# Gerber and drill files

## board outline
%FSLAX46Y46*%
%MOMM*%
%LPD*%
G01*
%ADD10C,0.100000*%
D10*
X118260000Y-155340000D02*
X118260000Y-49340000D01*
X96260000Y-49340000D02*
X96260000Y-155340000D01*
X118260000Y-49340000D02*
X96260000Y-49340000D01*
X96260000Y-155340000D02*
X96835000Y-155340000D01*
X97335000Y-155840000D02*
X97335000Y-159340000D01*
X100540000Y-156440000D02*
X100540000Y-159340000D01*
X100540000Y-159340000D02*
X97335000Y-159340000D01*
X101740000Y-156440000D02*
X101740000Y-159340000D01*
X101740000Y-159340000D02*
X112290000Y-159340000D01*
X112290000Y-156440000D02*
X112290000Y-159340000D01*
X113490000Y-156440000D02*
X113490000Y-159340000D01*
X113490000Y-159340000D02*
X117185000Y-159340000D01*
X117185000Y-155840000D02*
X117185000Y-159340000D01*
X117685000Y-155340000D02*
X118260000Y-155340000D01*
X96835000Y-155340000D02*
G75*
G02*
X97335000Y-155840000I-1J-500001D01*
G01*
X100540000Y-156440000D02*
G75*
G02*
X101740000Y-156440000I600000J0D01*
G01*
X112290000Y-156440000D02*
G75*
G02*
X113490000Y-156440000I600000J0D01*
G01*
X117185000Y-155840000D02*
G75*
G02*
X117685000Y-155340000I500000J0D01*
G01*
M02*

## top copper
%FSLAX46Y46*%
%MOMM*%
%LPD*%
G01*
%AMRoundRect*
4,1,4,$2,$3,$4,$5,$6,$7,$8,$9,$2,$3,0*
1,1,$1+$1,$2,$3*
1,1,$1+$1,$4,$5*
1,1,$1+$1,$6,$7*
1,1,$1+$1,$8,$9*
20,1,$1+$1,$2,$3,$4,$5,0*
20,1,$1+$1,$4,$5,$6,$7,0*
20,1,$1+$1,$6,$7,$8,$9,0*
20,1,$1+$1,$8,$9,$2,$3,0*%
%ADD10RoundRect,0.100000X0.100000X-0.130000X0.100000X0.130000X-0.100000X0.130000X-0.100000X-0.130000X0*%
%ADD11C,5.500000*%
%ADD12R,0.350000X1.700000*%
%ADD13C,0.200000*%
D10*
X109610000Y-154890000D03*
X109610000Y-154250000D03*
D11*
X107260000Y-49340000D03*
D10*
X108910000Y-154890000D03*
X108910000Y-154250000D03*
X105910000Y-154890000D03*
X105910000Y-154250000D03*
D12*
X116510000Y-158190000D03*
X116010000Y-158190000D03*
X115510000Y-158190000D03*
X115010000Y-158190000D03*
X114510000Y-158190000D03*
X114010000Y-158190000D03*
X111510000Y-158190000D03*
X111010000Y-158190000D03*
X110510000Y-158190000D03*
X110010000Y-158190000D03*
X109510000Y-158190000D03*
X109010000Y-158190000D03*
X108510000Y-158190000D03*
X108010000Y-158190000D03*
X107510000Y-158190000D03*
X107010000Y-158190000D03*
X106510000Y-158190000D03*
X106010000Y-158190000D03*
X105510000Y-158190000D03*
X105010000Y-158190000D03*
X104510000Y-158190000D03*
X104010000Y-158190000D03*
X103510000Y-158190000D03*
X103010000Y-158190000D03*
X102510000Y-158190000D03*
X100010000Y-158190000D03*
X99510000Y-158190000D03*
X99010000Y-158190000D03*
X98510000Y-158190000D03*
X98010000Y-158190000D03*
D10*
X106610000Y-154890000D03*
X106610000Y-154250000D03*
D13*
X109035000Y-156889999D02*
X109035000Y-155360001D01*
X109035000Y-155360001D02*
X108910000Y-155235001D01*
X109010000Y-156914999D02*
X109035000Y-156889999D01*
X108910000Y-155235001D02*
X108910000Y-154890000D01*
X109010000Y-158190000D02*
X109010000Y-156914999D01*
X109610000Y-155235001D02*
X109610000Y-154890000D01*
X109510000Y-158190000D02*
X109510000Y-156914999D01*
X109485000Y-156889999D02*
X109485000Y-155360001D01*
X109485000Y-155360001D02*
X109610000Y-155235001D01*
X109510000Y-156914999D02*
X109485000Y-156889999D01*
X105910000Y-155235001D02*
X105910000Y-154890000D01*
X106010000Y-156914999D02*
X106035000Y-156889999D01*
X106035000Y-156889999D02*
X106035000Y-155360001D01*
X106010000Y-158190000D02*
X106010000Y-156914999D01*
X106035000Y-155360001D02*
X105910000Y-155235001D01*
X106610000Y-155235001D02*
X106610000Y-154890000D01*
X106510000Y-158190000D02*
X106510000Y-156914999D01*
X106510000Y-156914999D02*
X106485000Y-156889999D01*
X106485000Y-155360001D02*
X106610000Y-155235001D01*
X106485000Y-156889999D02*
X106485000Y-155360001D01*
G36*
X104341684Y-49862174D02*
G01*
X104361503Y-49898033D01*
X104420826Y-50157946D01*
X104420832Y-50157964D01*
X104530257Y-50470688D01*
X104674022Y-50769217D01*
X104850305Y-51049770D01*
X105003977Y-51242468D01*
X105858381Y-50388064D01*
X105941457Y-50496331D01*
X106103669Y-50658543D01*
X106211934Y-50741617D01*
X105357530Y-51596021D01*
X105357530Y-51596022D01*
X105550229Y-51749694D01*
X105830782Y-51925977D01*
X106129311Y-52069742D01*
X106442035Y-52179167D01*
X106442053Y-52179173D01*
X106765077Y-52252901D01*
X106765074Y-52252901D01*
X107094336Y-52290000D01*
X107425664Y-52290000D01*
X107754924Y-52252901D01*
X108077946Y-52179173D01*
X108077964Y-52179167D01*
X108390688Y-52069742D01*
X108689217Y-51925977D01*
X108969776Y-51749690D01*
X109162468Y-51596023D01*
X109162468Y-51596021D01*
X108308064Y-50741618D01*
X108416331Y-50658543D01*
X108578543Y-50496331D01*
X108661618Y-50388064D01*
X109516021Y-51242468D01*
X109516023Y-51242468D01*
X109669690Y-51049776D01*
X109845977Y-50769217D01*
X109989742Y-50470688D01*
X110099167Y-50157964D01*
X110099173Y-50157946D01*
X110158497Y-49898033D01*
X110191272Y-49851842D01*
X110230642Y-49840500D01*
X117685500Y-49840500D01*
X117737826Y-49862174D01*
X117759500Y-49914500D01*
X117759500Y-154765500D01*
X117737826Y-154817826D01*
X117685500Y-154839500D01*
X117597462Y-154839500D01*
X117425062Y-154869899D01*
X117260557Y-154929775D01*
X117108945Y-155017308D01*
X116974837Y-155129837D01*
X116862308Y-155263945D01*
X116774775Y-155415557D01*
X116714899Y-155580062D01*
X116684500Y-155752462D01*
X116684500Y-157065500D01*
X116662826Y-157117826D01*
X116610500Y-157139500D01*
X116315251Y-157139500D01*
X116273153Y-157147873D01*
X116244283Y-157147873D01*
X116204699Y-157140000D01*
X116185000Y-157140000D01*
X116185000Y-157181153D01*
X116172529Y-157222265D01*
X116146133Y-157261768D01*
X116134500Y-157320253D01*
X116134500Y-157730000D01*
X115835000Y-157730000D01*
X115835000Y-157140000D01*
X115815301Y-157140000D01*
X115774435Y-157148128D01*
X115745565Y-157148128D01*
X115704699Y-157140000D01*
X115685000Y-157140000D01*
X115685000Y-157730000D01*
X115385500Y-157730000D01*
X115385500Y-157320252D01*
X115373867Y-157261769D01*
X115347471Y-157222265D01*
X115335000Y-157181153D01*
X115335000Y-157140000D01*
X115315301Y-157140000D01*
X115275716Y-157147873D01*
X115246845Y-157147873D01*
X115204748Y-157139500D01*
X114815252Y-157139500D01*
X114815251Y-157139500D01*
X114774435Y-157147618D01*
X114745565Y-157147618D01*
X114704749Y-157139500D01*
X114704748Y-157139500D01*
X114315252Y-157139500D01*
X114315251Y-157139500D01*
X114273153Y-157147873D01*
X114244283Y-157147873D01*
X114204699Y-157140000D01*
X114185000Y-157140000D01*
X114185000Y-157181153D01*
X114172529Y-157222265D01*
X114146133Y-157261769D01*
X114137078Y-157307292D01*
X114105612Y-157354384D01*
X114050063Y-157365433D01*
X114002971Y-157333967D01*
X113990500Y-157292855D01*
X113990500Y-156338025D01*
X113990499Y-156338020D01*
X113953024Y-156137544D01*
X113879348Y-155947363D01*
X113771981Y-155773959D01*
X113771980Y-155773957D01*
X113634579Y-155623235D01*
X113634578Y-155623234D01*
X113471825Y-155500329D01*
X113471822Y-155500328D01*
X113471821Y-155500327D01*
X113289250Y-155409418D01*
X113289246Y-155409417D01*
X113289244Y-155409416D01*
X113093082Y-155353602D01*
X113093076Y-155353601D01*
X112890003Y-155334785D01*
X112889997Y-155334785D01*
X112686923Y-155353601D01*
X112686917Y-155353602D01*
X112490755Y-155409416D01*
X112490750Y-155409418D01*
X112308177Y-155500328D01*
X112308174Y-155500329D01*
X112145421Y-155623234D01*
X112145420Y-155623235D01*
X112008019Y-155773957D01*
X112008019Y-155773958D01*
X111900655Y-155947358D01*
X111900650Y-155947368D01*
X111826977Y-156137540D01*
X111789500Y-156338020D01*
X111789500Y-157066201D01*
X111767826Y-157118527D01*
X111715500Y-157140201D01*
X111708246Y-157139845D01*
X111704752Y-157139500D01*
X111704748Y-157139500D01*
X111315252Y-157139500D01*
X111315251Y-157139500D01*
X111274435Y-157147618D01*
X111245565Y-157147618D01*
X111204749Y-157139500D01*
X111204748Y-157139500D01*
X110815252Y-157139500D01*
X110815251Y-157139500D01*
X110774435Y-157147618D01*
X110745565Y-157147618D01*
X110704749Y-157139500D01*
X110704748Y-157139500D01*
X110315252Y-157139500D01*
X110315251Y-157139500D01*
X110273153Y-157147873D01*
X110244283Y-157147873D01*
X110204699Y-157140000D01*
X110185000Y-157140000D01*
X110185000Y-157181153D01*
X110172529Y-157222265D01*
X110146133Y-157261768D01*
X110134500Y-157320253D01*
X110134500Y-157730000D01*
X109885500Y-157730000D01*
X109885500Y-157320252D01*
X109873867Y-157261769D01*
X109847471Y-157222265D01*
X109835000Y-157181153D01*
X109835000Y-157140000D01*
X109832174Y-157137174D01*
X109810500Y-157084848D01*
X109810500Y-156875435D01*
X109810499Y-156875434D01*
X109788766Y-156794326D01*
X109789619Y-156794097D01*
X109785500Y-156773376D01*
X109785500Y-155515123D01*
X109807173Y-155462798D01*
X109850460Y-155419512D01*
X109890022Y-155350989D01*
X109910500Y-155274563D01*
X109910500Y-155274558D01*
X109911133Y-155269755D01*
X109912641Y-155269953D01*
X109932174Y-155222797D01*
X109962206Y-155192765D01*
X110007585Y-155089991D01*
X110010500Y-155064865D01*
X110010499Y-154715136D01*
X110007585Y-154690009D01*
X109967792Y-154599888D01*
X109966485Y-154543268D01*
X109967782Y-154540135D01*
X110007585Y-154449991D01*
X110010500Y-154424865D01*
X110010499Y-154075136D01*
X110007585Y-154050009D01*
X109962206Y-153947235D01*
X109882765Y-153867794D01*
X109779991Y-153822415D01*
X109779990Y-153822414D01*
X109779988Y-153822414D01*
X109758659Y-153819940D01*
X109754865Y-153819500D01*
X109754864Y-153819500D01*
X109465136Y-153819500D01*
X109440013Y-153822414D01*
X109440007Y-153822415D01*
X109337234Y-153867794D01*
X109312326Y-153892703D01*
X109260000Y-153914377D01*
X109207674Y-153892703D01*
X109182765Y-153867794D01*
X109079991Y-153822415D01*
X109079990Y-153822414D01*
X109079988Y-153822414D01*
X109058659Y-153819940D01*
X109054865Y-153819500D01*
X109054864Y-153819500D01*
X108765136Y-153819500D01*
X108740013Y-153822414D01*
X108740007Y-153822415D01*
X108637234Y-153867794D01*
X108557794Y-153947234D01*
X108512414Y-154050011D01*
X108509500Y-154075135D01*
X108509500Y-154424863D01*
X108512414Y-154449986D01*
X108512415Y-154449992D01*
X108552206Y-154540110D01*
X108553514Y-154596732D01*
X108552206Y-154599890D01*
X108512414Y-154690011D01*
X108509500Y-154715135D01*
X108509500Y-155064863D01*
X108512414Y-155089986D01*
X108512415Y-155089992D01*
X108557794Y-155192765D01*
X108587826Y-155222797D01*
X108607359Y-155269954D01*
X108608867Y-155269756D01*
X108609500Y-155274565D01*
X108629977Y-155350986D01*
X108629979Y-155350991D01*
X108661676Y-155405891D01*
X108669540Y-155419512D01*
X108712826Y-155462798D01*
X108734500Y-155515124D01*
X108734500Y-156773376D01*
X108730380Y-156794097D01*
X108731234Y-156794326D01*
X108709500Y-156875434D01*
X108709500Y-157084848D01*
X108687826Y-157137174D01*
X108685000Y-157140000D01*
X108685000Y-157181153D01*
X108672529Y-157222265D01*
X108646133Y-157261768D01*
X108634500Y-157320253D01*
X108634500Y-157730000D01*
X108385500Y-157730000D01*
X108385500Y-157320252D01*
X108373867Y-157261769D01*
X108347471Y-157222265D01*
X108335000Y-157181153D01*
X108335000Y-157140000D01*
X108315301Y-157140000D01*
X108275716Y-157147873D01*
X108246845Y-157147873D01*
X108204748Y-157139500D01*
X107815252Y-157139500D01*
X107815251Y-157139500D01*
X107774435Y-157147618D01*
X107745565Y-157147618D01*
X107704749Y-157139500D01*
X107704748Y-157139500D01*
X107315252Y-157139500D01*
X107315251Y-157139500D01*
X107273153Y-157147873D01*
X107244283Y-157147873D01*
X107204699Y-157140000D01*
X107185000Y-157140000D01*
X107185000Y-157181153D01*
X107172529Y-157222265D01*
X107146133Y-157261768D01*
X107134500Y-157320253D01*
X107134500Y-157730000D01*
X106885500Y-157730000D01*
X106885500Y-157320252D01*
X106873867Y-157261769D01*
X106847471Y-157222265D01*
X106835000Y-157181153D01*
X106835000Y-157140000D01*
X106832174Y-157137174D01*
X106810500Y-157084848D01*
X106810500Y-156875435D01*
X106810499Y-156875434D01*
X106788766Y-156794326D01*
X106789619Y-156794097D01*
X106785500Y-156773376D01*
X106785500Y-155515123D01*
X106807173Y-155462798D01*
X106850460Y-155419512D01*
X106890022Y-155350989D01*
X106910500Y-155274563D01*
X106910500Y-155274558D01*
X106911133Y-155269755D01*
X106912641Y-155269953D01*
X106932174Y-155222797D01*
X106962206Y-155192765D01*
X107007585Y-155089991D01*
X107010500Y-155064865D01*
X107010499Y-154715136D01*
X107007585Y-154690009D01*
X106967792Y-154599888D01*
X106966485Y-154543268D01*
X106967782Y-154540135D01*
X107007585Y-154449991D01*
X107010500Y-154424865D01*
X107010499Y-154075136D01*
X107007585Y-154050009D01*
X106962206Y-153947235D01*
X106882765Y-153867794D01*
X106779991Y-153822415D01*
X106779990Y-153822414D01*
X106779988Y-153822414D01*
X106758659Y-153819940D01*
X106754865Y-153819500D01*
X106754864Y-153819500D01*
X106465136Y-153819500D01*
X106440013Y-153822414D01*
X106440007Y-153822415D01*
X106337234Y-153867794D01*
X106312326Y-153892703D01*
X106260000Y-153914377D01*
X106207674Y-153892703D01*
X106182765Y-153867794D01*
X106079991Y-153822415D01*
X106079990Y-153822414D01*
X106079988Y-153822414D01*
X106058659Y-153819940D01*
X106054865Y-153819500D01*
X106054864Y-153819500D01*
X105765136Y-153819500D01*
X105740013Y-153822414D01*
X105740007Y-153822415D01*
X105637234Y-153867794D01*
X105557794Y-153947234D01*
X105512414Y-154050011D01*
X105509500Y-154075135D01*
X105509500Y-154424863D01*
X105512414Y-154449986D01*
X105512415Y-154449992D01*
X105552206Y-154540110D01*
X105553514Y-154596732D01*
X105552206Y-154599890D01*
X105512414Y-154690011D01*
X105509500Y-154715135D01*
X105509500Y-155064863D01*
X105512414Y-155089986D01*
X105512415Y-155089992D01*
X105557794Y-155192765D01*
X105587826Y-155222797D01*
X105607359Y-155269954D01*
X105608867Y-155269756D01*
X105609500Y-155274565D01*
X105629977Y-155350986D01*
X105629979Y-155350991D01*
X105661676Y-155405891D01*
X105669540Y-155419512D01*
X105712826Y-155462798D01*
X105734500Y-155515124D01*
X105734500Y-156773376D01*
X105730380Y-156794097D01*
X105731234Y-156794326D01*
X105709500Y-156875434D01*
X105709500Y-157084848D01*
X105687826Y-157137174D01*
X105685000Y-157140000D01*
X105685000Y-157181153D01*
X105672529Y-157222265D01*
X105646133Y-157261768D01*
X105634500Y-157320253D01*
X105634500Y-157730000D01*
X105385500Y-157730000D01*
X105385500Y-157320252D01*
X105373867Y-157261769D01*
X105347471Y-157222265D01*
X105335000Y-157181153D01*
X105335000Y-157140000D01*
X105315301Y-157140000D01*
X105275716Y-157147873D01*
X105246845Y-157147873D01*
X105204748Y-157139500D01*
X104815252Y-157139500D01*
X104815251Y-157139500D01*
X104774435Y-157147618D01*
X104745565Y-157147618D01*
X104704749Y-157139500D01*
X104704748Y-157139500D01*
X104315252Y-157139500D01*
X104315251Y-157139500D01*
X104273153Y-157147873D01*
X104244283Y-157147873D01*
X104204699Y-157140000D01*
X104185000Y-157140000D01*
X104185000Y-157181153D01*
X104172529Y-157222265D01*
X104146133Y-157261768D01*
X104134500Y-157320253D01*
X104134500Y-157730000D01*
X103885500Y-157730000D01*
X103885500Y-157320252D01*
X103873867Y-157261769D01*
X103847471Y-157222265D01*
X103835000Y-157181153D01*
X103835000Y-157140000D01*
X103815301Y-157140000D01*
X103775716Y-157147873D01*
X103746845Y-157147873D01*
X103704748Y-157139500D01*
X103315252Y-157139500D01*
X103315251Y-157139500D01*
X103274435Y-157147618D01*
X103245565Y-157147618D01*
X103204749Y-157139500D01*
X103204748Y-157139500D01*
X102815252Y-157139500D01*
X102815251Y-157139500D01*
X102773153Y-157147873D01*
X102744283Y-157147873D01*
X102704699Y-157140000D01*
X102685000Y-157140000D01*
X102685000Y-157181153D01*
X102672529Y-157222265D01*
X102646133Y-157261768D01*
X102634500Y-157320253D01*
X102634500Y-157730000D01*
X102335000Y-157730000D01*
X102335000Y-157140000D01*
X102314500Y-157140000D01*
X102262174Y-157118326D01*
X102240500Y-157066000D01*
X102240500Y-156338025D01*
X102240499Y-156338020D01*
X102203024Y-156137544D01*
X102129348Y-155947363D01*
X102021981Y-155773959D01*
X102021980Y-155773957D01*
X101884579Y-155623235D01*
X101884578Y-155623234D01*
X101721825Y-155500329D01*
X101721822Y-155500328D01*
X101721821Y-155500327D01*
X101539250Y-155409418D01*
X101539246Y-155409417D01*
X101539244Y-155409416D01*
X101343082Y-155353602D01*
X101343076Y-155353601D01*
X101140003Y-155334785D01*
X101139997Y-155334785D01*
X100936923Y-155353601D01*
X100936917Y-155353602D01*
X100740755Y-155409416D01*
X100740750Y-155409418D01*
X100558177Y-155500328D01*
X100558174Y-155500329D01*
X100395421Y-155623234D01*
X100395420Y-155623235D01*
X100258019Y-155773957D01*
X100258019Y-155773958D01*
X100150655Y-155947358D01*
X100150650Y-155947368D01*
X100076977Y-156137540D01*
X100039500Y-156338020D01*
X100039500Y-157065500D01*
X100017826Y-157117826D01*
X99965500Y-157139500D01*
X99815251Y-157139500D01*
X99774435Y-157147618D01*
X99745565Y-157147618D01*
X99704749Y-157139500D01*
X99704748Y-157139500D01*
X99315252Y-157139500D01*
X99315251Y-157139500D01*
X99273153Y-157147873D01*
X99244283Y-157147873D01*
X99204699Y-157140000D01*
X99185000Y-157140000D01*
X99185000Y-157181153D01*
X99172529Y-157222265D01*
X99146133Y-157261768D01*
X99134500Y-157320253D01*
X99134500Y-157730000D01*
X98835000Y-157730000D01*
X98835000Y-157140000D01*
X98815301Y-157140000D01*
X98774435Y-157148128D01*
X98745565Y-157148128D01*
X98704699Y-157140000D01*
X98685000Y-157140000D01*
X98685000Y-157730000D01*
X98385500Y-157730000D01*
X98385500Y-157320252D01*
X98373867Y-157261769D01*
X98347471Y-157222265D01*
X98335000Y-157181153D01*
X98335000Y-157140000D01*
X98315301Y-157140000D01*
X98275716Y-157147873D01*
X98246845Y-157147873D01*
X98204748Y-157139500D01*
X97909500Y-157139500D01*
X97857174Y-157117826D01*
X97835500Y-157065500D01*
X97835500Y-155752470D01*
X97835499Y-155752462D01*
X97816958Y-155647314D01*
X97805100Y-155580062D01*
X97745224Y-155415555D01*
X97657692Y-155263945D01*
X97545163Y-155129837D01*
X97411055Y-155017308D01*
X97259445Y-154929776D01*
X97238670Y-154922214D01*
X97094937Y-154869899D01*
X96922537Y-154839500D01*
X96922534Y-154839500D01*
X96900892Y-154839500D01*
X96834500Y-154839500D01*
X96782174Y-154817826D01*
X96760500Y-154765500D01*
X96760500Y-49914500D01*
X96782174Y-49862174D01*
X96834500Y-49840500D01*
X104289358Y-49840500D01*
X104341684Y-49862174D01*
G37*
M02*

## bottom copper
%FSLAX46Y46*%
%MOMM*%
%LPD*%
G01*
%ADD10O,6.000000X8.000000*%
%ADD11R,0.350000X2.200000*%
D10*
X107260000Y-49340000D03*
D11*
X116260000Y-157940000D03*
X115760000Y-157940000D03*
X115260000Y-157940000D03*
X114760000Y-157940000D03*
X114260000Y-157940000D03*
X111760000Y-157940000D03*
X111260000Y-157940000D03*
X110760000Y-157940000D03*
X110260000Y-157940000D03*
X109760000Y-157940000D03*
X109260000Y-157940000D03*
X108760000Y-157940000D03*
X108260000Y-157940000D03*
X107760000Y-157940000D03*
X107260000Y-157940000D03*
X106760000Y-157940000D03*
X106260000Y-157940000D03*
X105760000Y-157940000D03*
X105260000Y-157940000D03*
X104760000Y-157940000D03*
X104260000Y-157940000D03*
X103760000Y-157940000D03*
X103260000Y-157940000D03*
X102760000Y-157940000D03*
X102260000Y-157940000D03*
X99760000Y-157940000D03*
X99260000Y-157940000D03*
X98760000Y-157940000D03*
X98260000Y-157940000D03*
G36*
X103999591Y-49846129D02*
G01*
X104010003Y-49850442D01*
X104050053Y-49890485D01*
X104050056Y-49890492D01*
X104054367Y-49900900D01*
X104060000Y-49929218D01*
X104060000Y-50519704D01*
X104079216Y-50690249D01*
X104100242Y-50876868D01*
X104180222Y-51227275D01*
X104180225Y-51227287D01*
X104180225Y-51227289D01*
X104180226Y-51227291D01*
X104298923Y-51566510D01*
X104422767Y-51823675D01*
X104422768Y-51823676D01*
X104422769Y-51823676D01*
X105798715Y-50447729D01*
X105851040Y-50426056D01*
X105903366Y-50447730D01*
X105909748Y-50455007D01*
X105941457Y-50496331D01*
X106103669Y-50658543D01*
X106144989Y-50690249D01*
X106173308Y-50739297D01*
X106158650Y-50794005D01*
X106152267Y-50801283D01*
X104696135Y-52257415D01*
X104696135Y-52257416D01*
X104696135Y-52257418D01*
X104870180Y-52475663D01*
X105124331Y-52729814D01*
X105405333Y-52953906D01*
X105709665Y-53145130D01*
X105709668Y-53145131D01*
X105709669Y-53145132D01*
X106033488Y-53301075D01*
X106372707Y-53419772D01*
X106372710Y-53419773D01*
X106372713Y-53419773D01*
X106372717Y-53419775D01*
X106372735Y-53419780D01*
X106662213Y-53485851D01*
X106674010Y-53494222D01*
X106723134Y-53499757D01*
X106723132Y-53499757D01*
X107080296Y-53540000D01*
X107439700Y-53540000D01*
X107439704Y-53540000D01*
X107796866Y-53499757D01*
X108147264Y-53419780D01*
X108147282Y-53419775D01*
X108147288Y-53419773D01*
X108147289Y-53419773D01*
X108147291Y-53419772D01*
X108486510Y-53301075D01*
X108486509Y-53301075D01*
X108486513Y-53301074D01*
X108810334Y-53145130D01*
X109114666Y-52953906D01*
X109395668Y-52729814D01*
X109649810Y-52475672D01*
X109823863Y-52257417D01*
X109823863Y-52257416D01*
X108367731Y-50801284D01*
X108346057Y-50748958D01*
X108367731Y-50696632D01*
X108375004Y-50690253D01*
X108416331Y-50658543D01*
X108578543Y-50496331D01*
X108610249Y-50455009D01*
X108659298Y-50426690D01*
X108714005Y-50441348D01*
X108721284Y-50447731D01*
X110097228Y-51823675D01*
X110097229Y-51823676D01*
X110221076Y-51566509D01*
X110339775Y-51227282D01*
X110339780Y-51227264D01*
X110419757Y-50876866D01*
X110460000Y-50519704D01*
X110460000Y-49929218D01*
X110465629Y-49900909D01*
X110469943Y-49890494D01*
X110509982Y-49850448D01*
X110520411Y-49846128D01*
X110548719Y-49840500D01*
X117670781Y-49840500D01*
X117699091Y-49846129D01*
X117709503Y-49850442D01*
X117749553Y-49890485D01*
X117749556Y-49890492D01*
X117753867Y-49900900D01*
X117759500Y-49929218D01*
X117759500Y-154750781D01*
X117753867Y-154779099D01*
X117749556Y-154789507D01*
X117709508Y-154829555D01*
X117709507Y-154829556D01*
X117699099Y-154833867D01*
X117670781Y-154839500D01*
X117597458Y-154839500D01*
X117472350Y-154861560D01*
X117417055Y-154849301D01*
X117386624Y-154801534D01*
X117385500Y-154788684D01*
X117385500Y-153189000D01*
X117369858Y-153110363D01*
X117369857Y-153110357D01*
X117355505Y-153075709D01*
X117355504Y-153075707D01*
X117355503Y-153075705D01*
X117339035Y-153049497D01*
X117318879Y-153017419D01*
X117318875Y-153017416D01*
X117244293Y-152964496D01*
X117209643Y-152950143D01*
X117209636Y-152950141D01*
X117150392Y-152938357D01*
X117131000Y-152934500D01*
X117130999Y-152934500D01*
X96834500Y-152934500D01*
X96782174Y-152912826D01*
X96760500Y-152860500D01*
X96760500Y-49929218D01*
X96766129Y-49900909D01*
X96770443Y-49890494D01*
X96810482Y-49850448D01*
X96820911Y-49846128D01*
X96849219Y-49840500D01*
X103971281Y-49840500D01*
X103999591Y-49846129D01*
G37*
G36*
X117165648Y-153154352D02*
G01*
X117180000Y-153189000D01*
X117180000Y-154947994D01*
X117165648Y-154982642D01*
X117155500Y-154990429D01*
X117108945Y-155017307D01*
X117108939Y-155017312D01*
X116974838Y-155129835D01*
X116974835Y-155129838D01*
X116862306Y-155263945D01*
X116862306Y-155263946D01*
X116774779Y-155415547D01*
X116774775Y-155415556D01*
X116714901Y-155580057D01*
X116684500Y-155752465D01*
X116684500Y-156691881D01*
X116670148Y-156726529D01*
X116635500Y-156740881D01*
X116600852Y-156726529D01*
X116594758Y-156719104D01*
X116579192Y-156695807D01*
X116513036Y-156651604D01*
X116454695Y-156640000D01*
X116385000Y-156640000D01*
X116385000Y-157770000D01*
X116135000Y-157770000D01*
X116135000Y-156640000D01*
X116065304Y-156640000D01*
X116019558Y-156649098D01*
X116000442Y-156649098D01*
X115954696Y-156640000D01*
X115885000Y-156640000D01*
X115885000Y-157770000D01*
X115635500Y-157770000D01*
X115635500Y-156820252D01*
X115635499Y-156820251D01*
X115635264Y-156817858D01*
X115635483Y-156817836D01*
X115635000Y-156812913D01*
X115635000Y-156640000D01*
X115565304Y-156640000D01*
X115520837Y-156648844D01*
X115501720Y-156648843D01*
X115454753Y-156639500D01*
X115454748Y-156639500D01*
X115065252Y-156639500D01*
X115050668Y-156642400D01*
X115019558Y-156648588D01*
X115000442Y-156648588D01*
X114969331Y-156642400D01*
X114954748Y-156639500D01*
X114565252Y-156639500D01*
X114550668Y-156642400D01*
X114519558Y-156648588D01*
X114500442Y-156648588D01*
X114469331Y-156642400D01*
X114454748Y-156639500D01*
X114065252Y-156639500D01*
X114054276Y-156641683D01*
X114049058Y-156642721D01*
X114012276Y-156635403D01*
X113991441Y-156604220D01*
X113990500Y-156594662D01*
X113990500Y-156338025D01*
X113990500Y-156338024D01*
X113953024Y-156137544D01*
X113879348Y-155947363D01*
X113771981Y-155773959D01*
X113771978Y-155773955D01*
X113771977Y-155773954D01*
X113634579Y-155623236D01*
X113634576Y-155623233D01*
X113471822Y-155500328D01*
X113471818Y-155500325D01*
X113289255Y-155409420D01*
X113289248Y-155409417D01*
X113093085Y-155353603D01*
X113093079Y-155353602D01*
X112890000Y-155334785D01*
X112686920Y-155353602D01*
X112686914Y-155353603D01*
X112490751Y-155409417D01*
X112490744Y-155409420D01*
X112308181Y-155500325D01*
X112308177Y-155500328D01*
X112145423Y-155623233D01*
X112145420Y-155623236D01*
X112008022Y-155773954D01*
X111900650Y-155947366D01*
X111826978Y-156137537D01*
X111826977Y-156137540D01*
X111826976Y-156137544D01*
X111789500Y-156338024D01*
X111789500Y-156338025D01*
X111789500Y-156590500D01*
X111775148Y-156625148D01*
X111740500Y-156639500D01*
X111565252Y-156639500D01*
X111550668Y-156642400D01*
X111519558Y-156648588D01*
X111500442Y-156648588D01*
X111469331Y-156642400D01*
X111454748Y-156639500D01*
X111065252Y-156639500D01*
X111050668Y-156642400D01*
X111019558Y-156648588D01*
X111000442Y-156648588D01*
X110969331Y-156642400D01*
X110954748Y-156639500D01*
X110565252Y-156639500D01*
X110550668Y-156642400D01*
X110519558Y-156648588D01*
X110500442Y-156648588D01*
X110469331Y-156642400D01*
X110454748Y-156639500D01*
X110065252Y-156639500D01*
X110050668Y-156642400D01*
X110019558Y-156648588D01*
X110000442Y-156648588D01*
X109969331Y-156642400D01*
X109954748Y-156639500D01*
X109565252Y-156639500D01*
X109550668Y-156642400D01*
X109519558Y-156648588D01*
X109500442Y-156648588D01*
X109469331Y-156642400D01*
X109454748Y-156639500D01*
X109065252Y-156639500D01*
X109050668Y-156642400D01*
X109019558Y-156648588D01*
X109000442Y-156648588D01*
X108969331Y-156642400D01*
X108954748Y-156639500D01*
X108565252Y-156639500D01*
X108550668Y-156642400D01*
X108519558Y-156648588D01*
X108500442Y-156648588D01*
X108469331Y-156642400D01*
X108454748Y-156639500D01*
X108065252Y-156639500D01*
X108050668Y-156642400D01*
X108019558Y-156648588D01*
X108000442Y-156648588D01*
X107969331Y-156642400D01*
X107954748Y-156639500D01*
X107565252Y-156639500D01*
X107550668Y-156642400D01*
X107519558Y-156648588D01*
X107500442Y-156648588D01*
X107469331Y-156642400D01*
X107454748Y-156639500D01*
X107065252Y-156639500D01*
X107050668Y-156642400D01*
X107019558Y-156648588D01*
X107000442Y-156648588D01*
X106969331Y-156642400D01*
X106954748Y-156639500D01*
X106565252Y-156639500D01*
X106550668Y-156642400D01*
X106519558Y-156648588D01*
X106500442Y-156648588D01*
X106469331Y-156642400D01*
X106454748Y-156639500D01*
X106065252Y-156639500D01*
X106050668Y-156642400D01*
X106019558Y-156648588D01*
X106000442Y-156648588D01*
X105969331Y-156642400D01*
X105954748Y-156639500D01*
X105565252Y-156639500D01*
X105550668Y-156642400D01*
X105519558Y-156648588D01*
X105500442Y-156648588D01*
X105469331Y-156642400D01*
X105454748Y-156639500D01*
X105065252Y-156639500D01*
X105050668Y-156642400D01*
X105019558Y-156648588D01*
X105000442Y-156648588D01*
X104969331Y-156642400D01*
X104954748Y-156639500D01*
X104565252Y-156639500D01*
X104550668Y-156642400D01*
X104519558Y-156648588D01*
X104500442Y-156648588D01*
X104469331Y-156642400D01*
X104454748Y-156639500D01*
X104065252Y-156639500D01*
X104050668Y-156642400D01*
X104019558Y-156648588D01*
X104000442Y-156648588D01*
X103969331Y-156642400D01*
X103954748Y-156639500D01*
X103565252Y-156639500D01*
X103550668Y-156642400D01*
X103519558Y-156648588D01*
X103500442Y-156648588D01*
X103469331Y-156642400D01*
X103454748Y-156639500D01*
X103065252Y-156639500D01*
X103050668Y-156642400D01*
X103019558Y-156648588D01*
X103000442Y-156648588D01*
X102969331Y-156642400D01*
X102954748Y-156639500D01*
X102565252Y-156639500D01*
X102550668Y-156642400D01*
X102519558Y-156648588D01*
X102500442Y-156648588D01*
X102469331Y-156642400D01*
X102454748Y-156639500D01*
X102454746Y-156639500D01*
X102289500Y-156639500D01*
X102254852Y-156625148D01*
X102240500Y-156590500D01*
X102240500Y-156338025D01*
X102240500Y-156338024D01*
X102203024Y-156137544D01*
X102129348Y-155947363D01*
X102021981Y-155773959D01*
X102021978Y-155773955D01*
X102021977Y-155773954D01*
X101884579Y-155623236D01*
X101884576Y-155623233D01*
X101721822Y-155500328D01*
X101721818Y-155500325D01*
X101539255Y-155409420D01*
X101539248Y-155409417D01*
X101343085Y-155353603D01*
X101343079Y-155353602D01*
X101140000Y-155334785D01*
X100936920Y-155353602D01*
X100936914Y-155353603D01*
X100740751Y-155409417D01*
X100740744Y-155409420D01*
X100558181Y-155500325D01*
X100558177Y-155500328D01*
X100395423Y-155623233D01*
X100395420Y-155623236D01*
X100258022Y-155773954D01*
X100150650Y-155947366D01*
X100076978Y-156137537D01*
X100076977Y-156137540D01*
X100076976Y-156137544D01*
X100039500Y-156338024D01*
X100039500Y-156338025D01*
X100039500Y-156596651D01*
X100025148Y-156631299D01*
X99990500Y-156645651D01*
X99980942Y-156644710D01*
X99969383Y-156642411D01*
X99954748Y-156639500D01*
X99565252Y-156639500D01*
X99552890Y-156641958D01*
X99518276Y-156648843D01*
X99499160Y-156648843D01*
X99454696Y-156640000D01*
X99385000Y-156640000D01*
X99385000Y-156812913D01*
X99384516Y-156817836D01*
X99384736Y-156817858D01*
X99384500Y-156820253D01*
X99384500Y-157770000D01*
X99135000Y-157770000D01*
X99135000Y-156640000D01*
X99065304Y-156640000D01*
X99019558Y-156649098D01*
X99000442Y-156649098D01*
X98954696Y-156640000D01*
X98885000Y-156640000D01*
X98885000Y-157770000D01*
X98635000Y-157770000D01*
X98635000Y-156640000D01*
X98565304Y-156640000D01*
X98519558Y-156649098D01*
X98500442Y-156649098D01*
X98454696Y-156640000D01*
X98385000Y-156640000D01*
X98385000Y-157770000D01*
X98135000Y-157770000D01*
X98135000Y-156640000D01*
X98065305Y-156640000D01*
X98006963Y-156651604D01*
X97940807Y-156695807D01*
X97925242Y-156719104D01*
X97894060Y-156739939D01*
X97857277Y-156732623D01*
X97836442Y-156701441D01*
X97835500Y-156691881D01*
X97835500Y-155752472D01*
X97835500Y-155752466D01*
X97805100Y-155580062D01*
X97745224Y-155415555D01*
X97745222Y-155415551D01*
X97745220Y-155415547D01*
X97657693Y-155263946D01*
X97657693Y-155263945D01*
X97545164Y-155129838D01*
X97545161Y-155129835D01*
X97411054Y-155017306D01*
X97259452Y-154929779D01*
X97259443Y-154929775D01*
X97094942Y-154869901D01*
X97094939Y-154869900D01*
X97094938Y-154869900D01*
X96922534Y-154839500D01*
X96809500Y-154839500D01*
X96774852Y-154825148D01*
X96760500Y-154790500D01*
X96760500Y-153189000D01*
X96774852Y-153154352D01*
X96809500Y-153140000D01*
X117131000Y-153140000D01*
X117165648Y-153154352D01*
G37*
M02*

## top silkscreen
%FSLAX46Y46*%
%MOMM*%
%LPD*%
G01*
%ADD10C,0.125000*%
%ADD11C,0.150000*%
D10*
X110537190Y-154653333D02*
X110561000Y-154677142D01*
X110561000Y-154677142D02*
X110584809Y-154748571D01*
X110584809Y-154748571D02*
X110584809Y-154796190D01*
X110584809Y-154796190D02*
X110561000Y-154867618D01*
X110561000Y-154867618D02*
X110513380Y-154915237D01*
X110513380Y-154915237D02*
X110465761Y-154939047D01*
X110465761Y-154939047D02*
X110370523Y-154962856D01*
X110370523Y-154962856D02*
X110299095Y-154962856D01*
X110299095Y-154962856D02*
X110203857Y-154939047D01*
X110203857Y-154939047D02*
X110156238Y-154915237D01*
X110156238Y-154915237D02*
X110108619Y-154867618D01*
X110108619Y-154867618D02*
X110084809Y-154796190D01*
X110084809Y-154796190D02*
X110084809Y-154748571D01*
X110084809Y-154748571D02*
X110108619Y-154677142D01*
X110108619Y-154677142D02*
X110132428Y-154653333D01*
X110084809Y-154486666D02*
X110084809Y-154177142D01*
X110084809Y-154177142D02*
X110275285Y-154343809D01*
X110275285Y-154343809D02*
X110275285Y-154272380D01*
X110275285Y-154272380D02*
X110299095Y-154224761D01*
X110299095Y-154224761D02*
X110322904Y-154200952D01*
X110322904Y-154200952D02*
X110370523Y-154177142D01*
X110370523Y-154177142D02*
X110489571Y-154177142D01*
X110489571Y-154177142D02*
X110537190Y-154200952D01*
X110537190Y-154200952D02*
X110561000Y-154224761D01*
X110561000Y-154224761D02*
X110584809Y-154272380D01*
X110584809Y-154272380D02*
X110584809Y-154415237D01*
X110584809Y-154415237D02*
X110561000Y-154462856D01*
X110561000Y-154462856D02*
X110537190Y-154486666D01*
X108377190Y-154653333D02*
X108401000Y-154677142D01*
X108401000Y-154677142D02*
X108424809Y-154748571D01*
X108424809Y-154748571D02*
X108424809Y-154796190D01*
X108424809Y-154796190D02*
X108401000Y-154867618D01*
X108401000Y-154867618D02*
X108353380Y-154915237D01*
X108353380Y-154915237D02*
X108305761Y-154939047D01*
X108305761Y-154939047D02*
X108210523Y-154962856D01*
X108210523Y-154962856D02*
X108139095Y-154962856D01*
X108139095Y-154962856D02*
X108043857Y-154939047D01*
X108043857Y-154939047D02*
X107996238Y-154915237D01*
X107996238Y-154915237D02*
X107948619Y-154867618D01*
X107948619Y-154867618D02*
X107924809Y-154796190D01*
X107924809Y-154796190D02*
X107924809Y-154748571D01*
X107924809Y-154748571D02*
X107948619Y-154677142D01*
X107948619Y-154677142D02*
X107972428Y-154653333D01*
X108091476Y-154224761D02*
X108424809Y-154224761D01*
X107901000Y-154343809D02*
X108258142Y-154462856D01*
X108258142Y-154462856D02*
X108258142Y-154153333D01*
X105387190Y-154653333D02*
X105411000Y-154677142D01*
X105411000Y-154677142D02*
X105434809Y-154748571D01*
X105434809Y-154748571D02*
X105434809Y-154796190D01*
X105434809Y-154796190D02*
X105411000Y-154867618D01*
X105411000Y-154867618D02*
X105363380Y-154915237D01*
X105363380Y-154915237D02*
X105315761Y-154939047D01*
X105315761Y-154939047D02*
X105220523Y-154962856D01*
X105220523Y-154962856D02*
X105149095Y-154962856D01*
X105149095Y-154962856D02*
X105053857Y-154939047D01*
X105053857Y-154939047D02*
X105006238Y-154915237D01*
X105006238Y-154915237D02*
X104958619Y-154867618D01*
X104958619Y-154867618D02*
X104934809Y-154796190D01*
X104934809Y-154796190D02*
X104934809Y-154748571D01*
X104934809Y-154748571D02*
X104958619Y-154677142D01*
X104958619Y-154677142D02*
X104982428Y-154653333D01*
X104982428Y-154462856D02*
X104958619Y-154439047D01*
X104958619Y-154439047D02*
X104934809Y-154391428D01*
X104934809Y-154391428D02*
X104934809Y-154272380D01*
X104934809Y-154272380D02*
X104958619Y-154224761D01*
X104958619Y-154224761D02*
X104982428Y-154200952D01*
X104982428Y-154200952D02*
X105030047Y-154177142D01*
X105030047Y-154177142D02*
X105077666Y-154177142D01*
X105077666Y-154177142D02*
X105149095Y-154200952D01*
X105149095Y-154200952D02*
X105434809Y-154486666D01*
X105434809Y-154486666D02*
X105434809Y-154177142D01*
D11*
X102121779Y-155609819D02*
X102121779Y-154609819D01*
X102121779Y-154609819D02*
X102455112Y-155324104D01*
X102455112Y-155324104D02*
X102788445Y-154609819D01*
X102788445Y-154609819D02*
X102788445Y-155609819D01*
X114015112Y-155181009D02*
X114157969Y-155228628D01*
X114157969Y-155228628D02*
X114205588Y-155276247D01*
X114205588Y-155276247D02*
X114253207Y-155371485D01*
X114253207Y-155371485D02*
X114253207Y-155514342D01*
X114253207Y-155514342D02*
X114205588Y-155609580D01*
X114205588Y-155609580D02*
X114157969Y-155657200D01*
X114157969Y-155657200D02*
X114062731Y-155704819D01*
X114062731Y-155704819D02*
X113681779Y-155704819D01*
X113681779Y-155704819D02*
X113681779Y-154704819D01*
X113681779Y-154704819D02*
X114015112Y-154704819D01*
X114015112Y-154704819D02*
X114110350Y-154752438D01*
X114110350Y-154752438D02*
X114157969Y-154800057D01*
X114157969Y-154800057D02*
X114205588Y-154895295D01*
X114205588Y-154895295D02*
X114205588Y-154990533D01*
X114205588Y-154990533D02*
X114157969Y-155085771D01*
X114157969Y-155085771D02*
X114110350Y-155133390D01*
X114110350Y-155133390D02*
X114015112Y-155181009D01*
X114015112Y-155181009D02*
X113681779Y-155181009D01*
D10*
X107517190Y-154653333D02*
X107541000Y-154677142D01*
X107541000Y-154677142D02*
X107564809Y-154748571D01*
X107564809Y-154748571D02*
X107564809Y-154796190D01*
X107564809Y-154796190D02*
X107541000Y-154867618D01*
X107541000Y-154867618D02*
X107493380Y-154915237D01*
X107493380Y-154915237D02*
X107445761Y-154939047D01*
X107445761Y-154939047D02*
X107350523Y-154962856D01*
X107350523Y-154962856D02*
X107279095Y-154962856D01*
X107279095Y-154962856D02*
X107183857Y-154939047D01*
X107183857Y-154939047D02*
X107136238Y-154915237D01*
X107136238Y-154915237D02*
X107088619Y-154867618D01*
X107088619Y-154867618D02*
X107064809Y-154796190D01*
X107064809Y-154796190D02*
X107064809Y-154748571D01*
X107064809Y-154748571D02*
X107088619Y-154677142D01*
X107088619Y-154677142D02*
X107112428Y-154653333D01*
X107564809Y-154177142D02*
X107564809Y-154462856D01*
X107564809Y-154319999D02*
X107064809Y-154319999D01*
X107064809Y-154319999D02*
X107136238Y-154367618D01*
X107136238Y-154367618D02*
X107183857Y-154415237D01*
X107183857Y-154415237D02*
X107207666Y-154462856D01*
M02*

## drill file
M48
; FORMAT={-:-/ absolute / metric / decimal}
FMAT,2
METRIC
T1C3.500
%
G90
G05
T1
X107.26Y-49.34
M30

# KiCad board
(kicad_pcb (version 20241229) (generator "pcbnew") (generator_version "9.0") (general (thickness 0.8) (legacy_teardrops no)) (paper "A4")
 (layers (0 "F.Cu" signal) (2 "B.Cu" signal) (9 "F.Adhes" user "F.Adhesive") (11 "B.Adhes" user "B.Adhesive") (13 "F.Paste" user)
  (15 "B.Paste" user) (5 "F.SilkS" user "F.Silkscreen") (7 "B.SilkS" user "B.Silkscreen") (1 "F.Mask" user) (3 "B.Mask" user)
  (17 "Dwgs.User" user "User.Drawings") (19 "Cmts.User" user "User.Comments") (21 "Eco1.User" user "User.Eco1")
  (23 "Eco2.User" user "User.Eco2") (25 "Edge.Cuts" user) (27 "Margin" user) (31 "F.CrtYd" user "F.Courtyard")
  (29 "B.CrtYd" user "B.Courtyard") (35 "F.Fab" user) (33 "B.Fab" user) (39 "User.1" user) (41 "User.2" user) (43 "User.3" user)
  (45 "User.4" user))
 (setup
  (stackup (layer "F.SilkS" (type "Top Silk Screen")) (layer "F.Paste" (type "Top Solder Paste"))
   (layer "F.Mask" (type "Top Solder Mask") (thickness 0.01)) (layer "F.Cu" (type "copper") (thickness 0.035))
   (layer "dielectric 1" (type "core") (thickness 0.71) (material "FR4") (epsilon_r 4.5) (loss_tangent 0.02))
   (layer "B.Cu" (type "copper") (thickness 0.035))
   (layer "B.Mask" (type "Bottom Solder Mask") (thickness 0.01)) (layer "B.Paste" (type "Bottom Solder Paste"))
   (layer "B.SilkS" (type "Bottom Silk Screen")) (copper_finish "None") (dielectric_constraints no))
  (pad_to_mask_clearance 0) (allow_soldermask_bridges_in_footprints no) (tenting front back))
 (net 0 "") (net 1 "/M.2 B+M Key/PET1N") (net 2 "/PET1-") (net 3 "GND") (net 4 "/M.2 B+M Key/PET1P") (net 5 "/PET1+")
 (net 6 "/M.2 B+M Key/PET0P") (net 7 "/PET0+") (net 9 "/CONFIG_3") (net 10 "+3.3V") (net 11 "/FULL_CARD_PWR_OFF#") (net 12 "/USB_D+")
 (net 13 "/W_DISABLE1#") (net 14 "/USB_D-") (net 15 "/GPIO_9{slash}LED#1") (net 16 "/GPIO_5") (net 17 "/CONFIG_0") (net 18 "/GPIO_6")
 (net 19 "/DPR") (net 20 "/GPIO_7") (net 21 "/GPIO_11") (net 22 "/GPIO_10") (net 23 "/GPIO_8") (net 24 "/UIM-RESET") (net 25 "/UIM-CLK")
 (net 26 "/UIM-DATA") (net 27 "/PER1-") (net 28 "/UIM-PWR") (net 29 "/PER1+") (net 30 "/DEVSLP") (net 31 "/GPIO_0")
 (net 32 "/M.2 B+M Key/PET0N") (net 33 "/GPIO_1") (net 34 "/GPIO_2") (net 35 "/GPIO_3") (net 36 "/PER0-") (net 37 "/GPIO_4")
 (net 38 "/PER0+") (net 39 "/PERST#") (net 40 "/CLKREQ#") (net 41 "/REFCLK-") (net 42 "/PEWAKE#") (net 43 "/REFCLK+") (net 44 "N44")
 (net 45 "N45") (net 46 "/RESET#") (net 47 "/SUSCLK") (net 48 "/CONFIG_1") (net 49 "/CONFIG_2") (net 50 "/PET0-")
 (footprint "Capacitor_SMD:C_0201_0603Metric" (layer "F.Cu") (at 109.61 154.57 90)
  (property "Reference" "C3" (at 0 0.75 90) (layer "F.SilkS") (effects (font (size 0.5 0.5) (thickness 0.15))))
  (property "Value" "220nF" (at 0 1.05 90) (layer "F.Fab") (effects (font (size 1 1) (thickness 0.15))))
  (pad "" smd roundrect (at -0.345 0 90) (size 0.318 0.36) (layers "F.Paste") (roundrect_rratio 0.25))
  (pad "" smd roundrect (at 0.345 0 90) (size 0.318 0.36) (layers "F.Paste") (roundrect_rratio 0.25))
  (pad "1" smd roundrect (at -0.32 0 90) (size 0.46 0.4) (layers "F.Cu" "F.Mask") (roundrect_rratio 0.25) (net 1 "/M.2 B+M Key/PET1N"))
  (pad "2" smd roundrect (at 0.32 0 90) (size 0.46 0.4) (layers "F.Cu" "F.Mask") (roundrect_rratio 0.25) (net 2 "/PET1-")))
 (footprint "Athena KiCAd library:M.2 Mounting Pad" (layer "F.Cu") (at 107.26 49.34)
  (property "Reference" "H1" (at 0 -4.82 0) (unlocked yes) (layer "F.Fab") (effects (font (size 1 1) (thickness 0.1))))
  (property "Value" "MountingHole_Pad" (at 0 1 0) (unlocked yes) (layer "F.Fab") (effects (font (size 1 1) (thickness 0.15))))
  (pad "1" thru_hole circle (at 0 0) (size 5.5 5.5) (drill 3.5) (layers "*.Cu" "*.Mask") (remove_unused_layers no) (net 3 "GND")
   (padstack (mode front_inner_back)
    (layer "Inner" (shape circle) (size 5.5 5.5) (zone_connect -1))
    (layer "B.Cu" (shape oval) (size 6 8) (thermal_bridge_angle 45) (zone_connect -1)))))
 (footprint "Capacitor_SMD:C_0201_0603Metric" (layer "F.Cu") (at 108.91 154.57 90)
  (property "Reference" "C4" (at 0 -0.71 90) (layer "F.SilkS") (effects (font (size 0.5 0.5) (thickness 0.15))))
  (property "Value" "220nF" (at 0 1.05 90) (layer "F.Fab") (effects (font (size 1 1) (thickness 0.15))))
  (pad "" smd roundrect (at -0.345 0 90) (size 0.318 0.36) (layers "F.Paste") (roundrect_rratio 0.25))
  (pad "" smd roundrect (at 0.345 0 90) (size 0.318 0.36) (layers "F.Paste") (roundrect_rratio 0.25))
  (pad "1" smd roundrect (at -0.32 0 90) (size 0.46 0.4) (layers "F.Cu" "F.Mask") (roundrect_rratio 0.25) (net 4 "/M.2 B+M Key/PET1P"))
  (pad "2" smd roundrect (at 0.32 0 90) (size 0.46 0.4) (layers "F.Cu" "F.Mask") (roundrect_rratio 0.25) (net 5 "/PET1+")))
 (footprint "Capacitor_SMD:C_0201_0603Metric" (layer "F.Cu") (at 105.91 154.57 90)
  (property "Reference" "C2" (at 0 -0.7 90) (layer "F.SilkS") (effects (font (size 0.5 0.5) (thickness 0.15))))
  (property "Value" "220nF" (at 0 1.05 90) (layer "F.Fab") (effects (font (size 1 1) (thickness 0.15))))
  (pad "" smd roundrect (at -0.345 0 90) (size 0.318 0.36) (layers "F.Paste") (roundrect_rratio 0.25))
  (pad "" smd roundrect (at 0.345 0 90) (size 0.318 0.36) (layers "F.Paste") (roundrect_rratio 0.25))
  (pad "1" smd roundrect (at -0.32 0 90) (size 0.46 0.4) (layers "F.Cu" "F.Mask") (roundrect_rratio 0.25) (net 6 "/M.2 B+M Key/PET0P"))
  (pad "2" smd roundrect (at 0.32 0 90) (size 0.46 0.4) (layers "F.Cu" "F.Mask") (roundrect_rratio 0.25) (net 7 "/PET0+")))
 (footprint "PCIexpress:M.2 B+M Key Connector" (layer "F.Cu") (at 107.26 158.23)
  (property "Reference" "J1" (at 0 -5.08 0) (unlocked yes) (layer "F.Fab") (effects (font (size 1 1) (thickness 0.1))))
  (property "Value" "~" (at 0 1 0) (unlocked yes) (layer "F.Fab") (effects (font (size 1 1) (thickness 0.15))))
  (fp_line (start -11 -2.89) (end -10.425 -2.89) (stroke (width 0.1) (type default)) (layer "Edge.Cuts") (net 8))
  (fp_line (start -9.925 -2.39) (end -9.925 1.11) (stroke (width 0.1) (type default)) (layer "Edge.Cuts") (net 8))
  (fp_line (start -6.72 -1.79) (end -6.72 1.11) (stroke (width 0.1) (type default)) (layer "Edge.Cuts") (net 8))
  (fp_line (start -6.72 1.11) (end -9.925 1.11) (stroke (width 0.1) (type default)) (layer "Edge.Cuts") (net 8))
  (fp_line (start -5.52 -1.79) (end -5.52 1.11) (stroke (width 0.1) (type default)) (layer "Edge.Cuts") (net 8))
  (fp_line (start -5.52 1.11) (end 5.03 1.11) (stroke (width 0.1) (type default)) (layer "Edge.Cuts") (net 8))
  (fp_line (start 5.03 -1.79) (end 5.03 1.11) (stroke (width 0.1) (type default)) (layer "Edge.Cuts") (net 8))
  (fp_line (start 6.23 -1.79) (end 6.23 1.11) (stroke (width 0.1) (type default)) (layer "Edge.Cuts") (net 8))
  (fp_line (start 6.23 1.11) (end 9.925 1.11) (stroke (width 0.1) (type default)) (layer "Edge.Cuts") (net 8))
  (fp_line (start 9.925 -2.39) (end 9.925 1.11) (stroke (width 0.1) (type default)) (layer "Edge.Cuts") (net 8))
  (fp_line (start 10.425 -2.89) (end 11 -2.89) (stroke (width 0.1) (type default)) (layer "Edge.Cuts") (net 8))
  (fp_arc (start -10.425 -2.89) (mid -10.071447 -2.743553) (end -9.925 -2.39) (stroke (width 0.1) (type default)) (layer "Edge.Cuts")
   (net 8))
  (fp_arc (start -6.72 -1.79) (mid -6.12 -2.39) (end -5.52 -1.79) (stroke (width 0.1) (type default)) (layer "Edge.Cuts") (net 8))
  (fp_arc (start 5.03 -1.79) (mid 5.63 -2.39) (end 6.23 -1.79) (stroke (width 0.1) (type default)) (layer "Edge.Cuts") (net 8))
  (fp_arc (start 9.925 -2.39) (mid 10.071447 -2.743553) (end 10.425 -2.89) (stroke (width 0.1) (type default)) (layer "Edge.Cuts") (net 8))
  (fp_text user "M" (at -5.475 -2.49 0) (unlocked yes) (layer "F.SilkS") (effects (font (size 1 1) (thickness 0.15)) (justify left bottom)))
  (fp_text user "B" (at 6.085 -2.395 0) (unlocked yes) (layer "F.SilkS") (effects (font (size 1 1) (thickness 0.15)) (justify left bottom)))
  (pad "1" smd rect (at 9.25 -0.04 180) (size 0.35 1.7) (layers "F.Cu") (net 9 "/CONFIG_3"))
  (pad "2" smd rect (at 9 -0.29 180) (size 0.35 2.2) (layers "B.Cu") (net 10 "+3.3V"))
  (pad "3" smd rect (at 8.75 -0.04 180) (size 0.35 1.7) (layers "F.Cu") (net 3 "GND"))
  (pad "4" smd rect (at 8.5 -0.29 180) (size 0.35 2.2) (layers "B.Cu") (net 10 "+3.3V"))
  (pad "5" smd rect (at 8.25 -0.04 180) (size 0.35 1.7) (layers "F.Cu") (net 3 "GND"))
  (pad "6" smd rect (at 8 -0.29 180) (size 0.35 2.2) (layers "B.Cu") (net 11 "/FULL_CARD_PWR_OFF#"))
  (pad "7" smd rect (at 7.75 -0.04 180) (size 0.35 1.7) (layers "F.Cu") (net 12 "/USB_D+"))
  (pad "8" smd rect (at 7.5 -0.29 180) (size 0.35 2.2) (layers "B.Cu") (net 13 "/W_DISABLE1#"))
  (pad "9" smd rect (at 7.25 -0.04 180) (size 0.35 1.7) (layers "F.Cu") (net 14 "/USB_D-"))
  (pad "10" smd rect (at 7 -0.29 180) (size 0.35 2.2) (layers "B.Cu") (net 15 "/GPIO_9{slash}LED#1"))
  (pad "11" smd rect (at 6.75 -0.04 180) (size 0.35 1.7) (layers "F.Cu") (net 3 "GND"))
  (pad "20" smd rect (at 4.5 -0.29 180) (size 0.35 2.2) (layers "B.Cu") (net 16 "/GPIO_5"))
  (pad "21" smd rect (at 4.25 -0.04 180) (size 0.35 1.7) (layers "F.Cu") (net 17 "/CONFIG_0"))
  (pad "22" smd rect (at 4 -0.29 180) (size 0.35 2.2) (layers "B.Cu") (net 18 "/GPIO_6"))
  (pad "23" smd rect (at 3.75 -0.04 180) (size 0.35 1.7) (layers "F.Cu") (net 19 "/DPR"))
  (pad "24" smd rect (at 3.5 -0.29 180) (size 0.35 2.2) (layers "B.Cu") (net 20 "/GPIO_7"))
  (pad "25" smd rect (at 3.25 -0.04 180) (size 0.35 1.7) (layers "F.Cu") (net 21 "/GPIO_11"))
  (pad "26" smd rect (at 3 -0.29 180) (size 0.35 2.2) (layers "B.Cu") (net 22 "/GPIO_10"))
  (pad "27" smd rect (at 2.75 -0.04 180) (size 0.35 1.7) (layers "F.Cu") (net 3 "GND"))
  (pad "28" smd rect (at 2.5 -0.29 180) (size 0.35 2.2) (layers "B.Cu") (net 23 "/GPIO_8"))
  (pad "29" smd rect (at 2.25 -0.04 180) (size 0.35 1.7) (layers "F.Cu") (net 1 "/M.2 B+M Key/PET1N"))
  (pad "30" smd rect (at 2 -0.29 180) (size 0.35 2.2) (layers "B.Cu") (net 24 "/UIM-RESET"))
  (pad "31" smd rect (at 1.75 -0.04 180) (size 0.35 1.7) (layers "F.Cu") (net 4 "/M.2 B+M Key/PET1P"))
  (pad "32" smd rect (at 1.5 -0.29 180) (size 0.35 2.2) (layers "B.Cu") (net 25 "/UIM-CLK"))
  (pad "33" smd rect (at 1.25 -0.04 180) (size 0.35 1.7) (layers "F.Cu") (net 3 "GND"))
  (pad "34" smd rect (at 1 -0.29 180) (size 0.35 2.2) (layers "B.Cu") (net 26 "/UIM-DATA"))
  (pad "35" smd rect (at 0.75 -0.04 180) (size 0.35 1.7) (layers "F.Cu") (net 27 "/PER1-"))
  (pad "36" smd rect (at 0.5 -0.29 180) (size 0.35 2.2) (layers "B.Cu") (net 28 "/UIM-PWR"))
  (pad "37" smd rect (at 0.25 -0.04 180) (size 0.35 1.7) (layers "F.Cu") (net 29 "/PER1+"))
  (pad "38" smd rect (at 0 -0.29 180) (size 0.35 2.2) (layers "B.Cu") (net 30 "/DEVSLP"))
  (pad "39" smd rect (at -0.25 -0.04 180) (size 0.35 1.7) (layers "F.Cu") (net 3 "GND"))
  (pad "40" smd rect (at -0.5 -0.29 180) (size 0.35 2.2) (layers "B.Cu") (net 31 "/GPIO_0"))
  (pad "41" smd rect (at -0.75 -0.04 180) (size 0.35 1.7) (layers "F.Cu") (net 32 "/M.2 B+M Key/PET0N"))
  (pad "42" smd rect (at -1 -0.29 180) (size 0.35 2.2) (layers "B.Cu") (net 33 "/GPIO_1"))
  (pad "43" smd rect (at -1.25 -0.04 180) (size 0.35 1.7) (layers "F.Cu") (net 6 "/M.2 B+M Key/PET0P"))
  (pad "44" smd rect (at -1.5 -0.29 180) (size 0.35 2.2) (layers "B.Cu") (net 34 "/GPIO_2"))
  (pad "45" smd rect (at -1.75 -0.04 180) (size 0.35 1.7) (layers "F.Cu") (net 3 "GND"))
  (pad "46" smd rect (at -2 -0.29 180) (size 0.35 2.2) (layers "B.Cu") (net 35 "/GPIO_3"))
  (pad "47" smd rect (at -2.25 -0.04 180) (size 0.35 1.7) (layers "F.Cu") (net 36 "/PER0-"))
  (pad "48" smd rect (at -2.5 -0.29 180) (size 0.35 2.2) (layers "B.Cu") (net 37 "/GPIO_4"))
  (pad "49" smd rect (at -2.75 -0.04 180) (size 0.35 1.7) (layers "F.Cu") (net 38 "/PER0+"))
  (pad "50" smd rect (at -3 -0.29 180) (size 0.35 2.2) (layers "B.Cu") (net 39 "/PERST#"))
  (pad "51" smd rect (at -3.25 -0.04 180) (size 0.35 1.7) (layers "F.Cu") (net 3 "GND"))
  (pad "52" smd rect (at -3.5 -0.29 180) (size 0.35 2.2) (layers "B.Cu") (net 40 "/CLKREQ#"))
  (pad "53" smd rect (at -3.75 -0.04 180) (size 0.35 1.7) (layers "F.Cu") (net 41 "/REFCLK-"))
  (pad "54" smd rect (at -4 -0.29 180) (size 0.35 2.2) (layers "B.Cu") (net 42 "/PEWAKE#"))
  (pad "55" smd rect (at -4.25 -0.04 180) (size 0.35 1.7) (layers "F.Cu") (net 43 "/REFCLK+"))
  (pad "56" smd rect (at -4.5 -0.29 180) (size 0.35 2.2) (layers "B.Cu") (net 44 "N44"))
  (pad "57" smd rect (at -4.75 -0.04 180) (size 0.35 1.7) (layers "F.Cu") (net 3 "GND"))
  (pad "58" smd rect (at -5 -0.29 180) (size 0.35 2.2) (layers "B.Cu") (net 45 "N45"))
  (pad "67" smd rect (at -7.25 -0.04 180) (size 0.35 1.7) (layers "F.Cu") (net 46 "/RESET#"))
  (pad "68" smd rect (at -7.5 -0.29 180) (size 0.35 2.2) (layers "B.Cu") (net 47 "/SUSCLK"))
  (pad "69" smd rect (at -7.75 -0.04 180) (size 0.35 1.7) (layers "F.Cu") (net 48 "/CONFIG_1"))
  (pad "70" smd rect (at -8 -0.29 180) (size 0.35 2.2) (layers "B.Cu") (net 10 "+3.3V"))
  (pad "71" smd rect (at -8.25 -0.04 180) (size 0.35 1.7) (layers "F.Cu") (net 3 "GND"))
  (pad "72" smd rect (at -8.5 -0.29 180) (size 0.35 2.2) (layers "B.Cu") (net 10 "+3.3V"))
  (pad "73" smd rect (at -8.75 -0.04 180) (size 0.35 1.7) (layers "F.Cu") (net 3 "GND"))
  (pad "74" smd rect (at -9 -0.29 180) (size 0.35 2.2) (layers "B.Cu") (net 10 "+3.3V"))
  (pad "75" smd rect (at -9.25 -0.04 180) (size 0.35 1.7) (layers "F.Cu") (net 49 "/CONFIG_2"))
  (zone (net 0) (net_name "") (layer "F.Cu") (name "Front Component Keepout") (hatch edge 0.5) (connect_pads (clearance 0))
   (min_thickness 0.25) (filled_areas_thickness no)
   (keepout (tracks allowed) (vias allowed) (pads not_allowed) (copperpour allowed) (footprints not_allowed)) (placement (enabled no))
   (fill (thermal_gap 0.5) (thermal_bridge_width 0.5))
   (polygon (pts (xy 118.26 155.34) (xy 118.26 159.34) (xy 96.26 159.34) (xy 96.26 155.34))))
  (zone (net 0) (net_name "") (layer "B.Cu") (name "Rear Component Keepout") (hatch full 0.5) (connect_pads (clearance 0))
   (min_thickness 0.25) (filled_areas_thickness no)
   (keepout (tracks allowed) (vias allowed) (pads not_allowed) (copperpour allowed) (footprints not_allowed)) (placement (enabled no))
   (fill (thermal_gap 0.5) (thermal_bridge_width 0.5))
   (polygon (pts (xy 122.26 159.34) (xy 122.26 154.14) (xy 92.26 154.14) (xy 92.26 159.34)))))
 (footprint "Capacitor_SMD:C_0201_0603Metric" (layer "F.Cu") (at 106.61 154.57 90)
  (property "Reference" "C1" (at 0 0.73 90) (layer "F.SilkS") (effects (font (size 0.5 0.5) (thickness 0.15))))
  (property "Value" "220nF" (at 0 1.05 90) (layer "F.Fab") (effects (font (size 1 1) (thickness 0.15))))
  (pad "" smd roundrect (at -0.345 0 90) (size 0.318 0.36) (layers "F.Paste") (roundrect_rratio 0.25))
  (pad "" smd roundrect (at 0.345 0 90) (size 0.318 0.36) (layers "F.Paste") (roundrect_rratio 0.25))
  (pad "1" smd roundrect (at -0.32 0 90) (size 0.46 0.4) (layers "F.Cu" "F.Mask") (roundrect_rratio 0.25) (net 32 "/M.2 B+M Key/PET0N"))
  (pad "2" smd roundrect (at 0.32 0 90) (size 0.46 0.4) (layers "F.Cu" "F.Mask") (roundrect_rratio 0.25) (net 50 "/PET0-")))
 (gr_line (start 118.26 155.34) (end 118.26 49.34) (stroke (width 0.1) (type default)) (layer "Edge.Cuts"))
 (gr_line (start 96.26 49.34) (end 96.26 155.34) (stroke (width 0.1) (type default)) (layer "Edge.Cuts"))
 (gr_line (start 118.26 49.34) (end 96.26 49.34) (stroke (width 0.1) (type default)) (layer "Edge.Cuts"))
 (segment (start 109.035 156.889999) (end 109.035 155.360001) (width 0.2) (layer "F.Cu") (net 4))
 (segment (start 109.035 155.360001) (end 108.91 155.235001) (width 0.2) (layer "F.Cu") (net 4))
 (segment (start 109.01 156.914999) (end 109.035 156.889999) (width 0.2) (layer "F.Cu") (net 4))
 (segment (start 108.91 155.235001) (end 108.91 154.89) (width 0.2) (layer "F.Cu") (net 4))
 (segment (start 109.01 158.19) (end 109.01 156.914999) (width 0.2) (layer "F.Cu") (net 4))
 (segment (start 109.61 155.235001) (end 109.61 154.89) (width 0.2) (layer "F.Cu") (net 1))
 (segment (start 109.51 158.19) (end 109.51 156.914999) (width 0.2) (layer "F.Cu") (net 1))
 (segment (start 109.485 156.889999) (end 109.485 155.360001) (width 0.2) (layer "F.Cu") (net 1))
 (segment (start 109.485 155.360001) (end 109.61 155.235001) (width 0.2) (layer "F.Cu") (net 1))
 (segment (start 109.51 156.914999) (end 109.485 156.889999) (width 0.2) (layer "F.Cu") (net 1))
 (segment (start 105.91 155.235001) (end 105.91 154.89) (width 0.2) (layer "F.Cu") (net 6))
 (segment (start 106.01 156.914999) (end 106.035 156.889999) (width 0.2) (layer "F.Cu") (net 6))
 (segment (start 106.035 156.889999) (end 106.035 155.360001) (width 0.2) (layer "F.Cu") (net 6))
 (segment (start 106.01 158.19) (end 106.01 156.914999) (width 0.2) (layer "F.Cu") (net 6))
 (segment (start 106.035 155.360001) (end 105.91 155.235001) (width 0.2) (layer "F.Cu") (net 6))
 (segment (start 106.61 155.235001) (end 106.61 154.89) (width 0.2) (layer "F.Cu") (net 32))
 (segment (start 106.51 158.19) (end 106.51 156.914999) (width 0.2) (layer "F.Cu") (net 32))
 (segment (start 106.51 156.914999) (end 106.485 156.889999) (width 0.2) (layer "F.Cu") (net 32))
 (segment (start 106.485 155.360001) (end 106.61 155.235001) (width 0.2) (layer "F.Cu") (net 32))
 (segment (start 106.485 156.889999) (end 106.485 155.360001) (width 0.2) (layer "F.Cu") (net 32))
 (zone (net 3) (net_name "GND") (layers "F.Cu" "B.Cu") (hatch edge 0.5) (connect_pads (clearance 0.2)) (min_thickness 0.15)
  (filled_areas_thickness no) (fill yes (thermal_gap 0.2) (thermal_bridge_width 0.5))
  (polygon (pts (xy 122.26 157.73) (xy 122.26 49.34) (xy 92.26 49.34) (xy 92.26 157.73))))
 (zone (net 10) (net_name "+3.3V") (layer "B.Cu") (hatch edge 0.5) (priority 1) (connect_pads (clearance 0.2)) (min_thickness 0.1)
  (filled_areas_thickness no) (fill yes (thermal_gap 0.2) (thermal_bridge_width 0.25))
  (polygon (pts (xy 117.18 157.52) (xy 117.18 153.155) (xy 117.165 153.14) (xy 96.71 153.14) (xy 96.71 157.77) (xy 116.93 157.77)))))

